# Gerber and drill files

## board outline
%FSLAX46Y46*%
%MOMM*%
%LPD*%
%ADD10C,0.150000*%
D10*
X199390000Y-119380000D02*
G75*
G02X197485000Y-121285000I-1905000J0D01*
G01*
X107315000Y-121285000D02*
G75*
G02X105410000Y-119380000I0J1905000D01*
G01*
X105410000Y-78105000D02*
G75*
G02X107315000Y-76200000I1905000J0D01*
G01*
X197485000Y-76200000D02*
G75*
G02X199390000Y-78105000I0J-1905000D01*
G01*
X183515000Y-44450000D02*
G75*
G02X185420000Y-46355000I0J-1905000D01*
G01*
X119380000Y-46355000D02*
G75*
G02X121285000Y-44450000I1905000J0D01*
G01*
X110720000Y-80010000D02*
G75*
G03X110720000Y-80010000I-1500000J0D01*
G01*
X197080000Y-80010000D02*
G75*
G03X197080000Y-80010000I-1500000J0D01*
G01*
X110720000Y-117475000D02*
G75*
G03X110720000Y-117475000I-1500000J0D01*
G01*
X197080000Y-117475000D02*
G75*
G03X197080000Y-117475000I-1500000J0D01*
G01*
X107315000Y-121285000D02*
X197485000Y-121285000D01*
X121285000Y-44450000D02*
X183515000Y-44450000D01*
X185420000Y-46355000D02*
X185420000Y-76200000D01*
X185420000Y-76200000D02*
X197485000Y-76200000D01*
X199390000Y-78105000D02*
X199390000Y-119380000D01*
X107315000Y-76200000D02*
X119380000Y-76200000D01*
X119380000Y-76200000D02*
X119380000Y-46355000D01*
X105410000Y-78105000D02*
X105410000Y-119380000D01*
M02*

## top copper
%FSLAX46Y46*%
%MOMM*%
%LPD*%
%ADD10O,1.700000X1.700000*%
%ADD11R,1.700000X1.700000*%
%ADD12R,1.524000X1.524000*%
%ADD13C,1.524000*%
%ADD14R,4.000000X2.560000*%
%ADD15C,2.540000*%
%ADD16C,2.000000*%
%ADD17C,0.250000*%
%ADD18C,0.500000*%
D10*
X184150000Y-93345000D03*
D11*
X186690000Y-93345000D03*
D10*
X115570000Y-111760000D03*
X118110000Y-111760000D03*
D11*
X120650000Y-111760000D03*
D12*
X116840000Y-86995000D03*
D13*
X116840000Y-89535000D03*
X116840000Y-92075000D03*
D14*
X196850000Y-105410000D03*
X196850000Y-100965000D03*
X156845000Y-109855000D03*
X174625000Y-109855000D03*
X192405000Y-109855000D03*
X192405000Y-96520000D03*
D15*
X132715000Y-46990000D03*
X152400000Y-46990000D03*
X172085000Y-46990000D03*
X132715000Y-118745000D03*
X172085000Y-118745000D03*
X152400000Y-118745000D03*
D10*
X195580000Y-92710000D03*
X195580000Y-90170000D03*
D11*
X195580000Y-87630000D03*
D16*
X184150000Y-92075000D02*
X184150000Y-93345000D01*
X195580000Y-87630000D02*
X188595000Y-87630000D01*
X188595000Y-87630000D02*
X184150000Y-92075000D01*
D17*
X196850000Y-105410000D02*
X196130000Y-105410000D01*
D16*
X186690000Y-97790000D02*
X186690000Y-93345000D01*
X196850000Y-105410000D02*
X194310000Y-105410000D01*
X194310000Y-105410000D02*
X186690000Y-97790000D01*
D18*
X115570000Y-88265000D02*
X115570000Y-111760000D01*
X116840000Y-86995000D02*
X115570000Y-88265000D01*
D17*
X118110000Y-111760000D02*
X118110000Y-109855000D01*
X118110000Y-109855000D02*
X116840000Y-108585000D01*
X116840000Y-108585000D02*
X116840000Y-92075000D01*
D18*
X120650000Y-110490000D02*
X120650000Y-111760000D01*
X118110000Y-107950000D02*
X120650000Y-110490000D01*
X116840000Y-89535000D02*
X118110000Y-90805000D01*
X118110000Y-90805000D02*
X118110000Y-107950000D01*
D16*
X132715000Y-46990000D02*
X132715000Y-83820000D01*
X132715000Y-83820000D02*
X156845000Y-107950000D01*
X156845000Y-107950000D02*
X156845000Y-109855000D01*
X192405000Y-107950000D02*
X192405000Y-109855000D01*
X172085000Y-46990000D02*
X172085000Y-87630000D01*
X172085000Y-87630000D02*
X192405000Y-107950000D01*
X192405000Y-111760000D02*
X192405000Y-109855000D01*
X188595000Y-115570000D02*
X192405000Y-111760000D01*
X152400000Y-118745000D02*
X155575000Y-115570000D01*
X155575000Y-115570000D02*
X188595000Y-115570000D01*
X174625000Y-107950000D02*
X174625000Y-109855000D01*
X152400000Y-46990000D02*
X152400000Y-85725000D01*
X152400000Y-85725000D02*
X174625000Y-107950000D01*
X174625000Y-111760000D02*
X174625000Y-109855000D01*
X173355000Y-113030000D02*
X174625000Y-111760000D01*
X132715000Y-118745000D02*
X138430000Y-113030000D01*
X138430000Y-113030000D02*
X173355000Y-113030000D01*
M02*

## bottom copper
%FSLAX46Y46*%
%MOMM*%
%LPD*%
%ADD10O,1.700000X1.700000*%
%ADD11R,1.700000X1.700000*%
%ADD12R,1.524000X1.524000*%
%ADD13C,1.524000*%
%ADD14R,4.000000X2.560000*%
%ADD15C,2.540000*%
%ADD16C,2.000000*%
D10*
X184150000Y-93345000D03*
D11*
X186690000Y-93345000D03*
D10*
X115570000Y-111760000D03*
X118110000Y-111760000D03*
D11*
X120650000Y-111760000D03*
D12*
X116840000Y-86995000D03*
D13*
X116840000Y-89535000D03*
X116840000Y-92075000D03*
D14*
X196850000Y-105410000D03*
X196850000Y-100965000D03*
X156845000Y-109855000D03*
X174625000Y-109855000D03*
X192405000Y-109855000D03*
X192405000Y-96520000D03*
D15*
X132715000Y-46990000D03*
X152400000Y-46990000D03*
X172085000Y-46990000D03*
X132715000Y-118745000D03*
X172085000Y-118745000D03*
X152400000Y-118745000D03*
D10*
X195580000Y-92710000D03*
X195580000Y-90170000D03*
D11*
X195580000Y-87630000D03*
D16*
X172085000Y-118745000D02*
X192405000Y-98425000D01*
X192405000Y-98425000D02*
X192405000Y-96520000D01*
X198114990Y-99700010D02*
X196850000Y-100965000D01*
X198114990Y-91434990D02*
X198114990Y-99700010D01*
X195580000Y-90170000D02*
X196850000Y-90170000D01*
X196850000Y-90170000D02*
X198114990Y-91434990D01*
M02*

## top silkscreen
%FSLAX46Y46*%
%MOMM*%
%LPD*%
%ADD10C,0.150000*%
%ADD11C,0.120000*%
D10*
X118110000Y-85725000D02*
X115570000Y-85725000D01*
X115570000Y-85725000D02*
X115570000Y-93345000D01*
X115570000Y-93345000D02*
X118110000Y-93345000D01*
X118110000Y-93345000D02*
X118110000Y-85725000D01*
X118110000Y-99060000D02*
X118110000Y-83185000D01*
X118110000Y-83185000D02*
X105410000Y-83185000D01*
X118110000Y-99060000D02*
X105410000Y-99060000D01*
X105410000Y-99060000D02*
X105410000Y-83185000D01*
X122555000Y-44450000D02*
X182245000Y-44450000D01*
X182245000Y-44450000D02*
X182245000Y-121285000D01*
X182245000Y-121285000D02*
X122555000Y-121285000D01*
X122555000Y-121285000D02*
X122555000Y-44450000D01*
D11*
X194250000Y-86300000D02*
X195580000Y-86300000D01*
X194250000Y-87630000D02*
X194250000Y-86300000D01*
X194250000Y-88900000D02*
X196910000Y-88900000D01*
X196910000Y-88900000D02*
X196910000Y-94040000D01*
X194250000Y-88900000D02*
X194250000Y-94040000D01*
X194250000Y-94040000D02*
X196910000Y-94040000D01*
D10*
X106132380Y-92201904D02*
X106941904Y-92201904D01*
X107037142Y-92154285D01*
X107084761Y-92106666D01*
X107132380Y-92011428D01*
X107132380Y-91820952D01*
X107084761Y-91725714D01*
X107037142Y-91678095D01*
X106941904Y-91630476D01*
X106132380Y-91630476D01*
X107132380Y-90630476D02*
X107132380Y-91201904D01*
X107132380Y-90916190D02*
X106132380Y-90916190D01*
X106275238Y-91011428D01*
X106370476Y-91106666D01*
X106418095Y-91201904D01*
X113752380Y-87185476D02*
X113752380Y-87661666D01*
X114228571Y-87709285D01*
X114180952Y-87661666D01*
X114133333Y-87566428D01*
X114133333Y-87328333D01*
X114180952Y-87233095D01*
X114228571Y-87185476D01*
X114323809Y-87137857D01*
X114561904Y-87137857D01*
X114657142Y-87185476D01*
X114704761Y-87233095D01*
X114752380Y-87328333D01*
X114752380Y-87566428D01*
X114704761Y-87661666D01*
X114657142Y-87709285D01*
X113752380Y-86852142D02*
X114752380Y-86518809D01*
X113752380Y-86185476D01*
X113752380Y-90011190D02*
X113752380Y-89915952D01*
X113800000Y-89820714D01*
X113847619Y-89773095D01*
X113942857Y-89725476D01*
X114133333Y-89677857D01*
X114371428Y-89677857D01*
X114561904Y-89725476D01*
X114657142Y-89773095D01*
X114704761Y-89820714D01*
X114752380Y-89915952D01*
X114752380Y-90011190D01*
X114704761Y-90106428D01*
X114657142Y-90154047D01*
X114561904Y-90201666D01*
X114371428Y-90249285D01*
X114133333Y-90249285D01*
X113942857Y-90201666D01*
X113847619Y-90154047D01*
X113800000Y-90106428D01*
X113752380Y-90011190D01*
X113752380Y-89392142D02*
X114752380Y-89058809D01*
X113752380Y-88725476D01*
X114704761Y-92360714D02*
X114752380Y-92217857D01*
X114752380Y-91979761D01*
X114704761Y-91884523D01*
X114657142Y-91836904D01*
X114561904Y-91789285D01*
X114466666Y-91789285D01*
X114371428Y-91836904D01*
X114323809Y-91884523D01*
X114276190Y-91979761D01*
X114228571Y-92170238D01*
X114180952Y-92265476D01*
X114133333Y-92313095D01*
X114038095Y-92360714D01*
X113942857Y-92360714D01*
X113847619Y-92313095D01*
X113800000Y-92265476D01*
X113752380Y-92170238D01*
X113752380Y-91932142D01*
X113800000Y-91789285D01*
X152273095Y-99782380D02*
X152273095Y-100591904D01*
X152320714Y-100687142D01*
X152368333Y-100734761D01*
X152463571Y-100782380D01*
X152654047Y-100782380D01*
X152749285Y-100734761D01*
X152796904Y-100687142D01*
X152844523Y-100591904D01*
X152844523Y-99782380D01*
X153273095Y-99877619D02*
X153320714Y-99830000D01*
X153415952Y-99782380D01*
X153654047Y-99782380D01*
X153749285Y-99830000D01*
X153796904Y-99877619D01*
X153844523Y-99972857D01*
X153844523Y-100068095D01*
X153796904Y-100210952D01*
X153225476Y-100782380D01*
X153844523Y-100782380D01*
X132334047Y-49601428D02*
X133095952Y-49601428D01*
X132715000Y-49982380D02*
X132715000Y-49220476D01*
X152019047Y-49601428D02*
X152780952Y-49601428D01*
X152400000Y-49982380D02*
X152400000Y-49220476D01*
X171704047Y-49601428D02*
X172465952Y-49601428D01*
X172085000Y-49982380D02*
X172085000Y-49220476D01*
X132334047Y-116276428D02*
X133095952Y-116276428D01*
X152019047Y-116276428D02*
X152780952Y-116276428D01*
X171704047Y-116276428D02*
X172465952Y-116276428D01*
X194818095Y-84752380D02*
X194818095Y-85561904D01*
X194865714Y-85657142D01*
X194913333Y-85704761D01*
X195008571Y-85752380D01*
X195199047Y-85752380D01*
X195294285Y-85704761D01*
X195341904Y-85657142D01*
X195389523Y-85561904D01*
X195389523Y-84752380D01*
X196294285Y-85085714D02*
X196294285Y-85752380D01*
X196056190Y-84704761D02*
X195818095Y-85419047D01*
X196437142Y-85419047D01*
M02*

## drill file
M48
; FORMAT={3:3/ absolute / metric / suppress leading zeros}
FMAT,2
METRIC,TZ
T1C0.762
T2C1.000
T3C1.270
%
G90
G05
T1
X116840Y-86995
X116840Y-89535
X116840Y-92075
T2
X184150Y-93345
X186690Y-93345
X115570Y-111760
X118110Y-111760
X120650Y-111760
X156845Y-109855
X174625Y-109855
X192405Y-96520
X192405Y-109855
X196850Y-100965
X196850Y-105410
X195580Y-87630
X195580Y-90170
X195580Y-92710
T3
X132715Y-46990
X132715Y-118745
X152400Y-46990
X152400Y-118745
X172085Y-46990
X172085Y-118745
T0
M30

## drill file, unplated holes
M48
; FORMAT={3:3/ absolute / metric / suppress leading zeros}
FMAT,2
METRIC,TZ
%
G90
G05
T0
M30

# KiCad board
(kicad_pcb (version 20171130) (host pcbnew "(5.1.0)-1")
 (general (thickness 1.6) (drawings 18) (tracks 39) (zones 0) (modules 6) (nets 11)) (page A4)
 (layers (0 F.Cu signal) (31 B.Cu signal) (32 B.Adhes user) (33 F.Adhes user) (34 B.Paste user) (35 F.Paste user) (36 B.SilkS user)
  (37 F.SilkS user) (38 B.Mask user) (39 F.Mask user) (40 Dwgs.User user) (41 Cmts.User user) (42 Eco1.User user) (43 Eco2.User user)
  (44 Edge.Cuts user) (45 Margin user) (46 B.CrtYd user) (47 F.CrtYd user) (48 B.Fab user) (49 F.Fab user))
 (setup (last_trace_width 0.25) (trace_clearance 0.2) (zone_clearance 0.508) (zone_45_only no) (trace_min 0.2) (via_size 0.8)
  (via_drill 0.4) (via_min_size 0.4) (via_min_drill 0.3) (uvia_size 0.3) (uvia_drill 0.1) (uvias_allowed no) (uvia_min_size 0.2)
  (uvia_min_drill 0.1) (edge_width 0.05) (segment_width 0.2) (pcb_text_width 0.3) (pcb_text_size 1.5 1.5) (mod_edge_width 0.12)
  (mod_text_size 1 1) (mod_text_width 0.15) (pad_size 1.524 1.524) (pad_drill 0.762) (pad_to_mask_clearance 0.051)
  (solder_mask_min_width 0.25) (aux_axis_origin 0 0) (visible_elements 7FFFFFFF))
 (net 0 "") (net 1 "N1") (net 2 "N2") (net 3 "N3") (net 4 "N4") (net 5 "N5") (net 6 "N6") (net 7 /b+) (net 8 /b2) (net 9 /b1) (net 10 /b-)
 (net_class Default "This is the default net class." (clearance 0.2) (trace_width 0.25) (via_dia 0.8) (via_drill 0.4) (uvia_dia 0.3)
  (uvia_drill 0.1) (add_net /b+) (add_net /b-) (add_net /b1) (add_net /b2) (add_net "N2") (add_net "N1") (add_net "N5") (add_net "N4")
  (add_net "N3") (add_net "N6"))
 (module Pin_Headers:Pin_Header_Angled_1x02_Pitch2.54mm (layer B.Cu) (at 186.69 93.345 90)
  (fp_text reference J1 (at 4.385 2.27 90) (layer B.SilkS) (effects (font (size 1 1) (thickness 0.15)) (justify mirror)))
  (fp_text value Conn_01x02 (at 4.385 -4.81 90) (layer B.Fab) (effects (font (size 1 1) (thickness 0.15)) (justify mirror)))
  (pad 2 thru_hole oval (at 0 -2.54 90) (size 1.7 1.7) (drill 1) (layers *.Cu *.Mask) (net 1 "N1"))
  (pad 1 thru_hole rect (at 0 0 90) (size 1.7 1.7) (drill 1) (layers *.Cu *.Mask) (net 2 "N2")))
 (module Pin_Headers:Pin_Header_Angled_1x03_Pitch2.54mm (layer B.Cu) (at 120.65 111.76 90)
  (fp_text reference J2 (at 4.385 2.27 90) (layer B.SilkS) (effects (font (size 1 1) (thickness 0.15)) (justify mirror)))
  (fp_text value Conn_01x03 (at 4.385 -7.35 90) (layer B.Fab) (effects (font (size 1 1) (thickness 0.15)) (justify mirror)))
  (pad 3 thru_hole oval (at 0 -5.08 90) (size 1.7 1.7) (drill 1) (layers *.Cu *.Mask) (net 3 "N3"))
  (pad 2 thru_hole oval (at 0 -2.54 90) (size 1.7 1.7) (drill 1) (layers *.Cu *.Mask) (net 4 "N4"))
  (pad 1 thru_hole rect (at 0 0 90) (size 1.7 1.7) (drill 1) (layers *.Cu *.Mask) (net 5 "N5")))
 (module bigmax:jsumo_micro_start (layer F.Cu) (at 116.84 86.995 270)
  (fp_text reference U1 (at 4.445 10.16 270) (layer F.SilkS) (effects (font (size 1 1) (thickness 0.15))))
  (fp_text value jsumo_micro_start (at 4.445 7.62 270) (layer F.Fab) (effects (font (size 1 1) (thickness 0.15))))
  (fp_line (start -1.27 -1.27) (end -1.27 1.27) (layer F.SilkS) (width 0.15))
  (fp_line (start -1.27 1.27) (end 6.35 1.27) (layer F.SilkS) (width 0.15))
  (fp_line (start 6.35 1.27) (end 6.35 -1.27) (layer F.SilkS) (width 0.15))
  (fp_line (start 6.35 -1.27) (end -1.27 -1.27) (layer F.SilkS) (width 0.15))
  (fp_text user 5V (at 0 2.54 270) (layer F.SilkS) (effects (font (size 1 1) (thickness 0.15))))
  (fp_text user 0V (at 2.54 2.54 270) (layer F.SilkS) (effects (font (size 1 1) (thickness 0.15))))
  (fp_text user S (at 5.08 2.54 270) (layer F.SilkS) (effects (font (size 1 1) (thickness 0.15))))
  (fp_line (start 12.065 -1.27) (end -3.81 -1.27) (layer F.SilkS) (width 0.15))
  (fp_line (start -3.81 -1.27) (end -3.81 11.43) (layer F.SilkS) (width 0.15))
  (fp_line (start 12.065 -1.27) (end 12.065 11.43) (layer F.SilkS) (width 0.15))
  (fp_line (start 12.065 11.43) (end -3.81 11.43) (layer F.SilkS) (width 0.15))
  (pad 1 thru_hole rect (at 0 0 270) (size 1.524 1.524) (drill 0.762) (layers *.Cu *.Mask) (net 3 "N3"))
  (pad 2 thru_hole circle (at 2.54 0 270) (size 1.524 1.524) (drill 0.762) (layers *.Cu *.Mask) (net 5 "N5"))
  (pad 3 thru_hole circle (at 5.08 0 270) (size 1.524 1.524) (drill 0.762) (layers *.Cu *.Mask) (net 4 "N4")))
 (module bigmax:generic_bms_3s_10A (layer B.Cu) (at 196.85 100.965)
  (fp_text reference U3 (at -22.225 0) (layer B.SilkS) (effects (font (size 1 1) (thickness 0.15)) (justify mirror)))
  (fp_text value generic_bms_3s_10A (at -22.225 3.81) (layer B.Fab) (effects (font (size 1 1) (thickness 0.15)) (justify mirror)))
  (pad 2 thru_hole rect (at 0 4.445) (size 4 2.56) (drill 1) (layers *.Cu *.Mask) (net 2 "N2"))
  (pad 1 thru_hole rect (at 0 0) (size 4 2.56) (drill 1) (layers *.Cu *.Mask) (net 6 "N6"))
  (pad 3 thru_hole rect (at -40.005 8.89) (size 4 2.56) (drill 1) (layers *.Cu *.Mask) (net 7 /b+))
  (pad 5 thru_hole rect (at -22.225 8.89) (size 4 2.56) (drill 1) (layers *.Cu *.Mask) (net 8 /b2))
  (pad 4 thru_hole rect (at -4.445 8.89) (size 4 2.56) (drill 1) (layers *.Cu *.Mask) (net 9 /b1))
  (pad 6 thru_hole rect (at -4.445 -4.445) (size 4 2.56) (drill 1) (layers *.Cu *.Mask) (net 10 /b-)))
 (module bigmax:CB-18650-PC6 (layer F.Cu) (at 132.715 46.99)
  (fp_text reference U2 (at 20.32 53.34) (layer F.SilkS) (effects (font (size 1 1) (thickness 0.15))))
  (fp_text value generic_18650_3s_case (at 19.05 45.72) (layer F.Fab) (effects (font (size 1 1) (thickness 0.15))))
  (fp_line (start -10.16 -2.54) (end 49.53 -2.54) (layer F.SilkS) (width 0.15))
  (fp_line (start 49.53 -2.54) (end 49.53 74.295) (layer F.SilkS) (width 0.15))
  (fp_line (start 49.53 74.295) (end -10.16 74.295) (layer F.SilkS) (width 0.15))
  (fp_line (start -10.16 74.295) (end -10.16 -2.54) (layer F.SilkS) (width 0.15))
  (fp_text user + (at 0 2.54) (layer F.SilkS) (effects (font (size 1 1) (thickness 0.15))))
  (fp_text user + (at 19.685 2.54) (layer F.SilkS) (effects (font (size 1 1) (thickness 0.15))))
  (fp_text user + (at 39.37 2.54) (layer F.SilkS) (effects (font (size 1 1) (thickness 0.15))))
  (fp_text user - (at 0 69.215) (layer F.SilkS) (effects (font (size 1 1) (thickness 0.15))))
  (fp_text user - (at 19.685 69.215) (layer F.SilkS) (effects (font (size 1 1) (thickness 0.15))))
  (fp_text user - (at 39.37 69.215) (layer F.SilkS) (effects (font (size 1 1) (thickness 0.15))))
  (pad 1 thru_hole circle (at 0 0) (size 2.54 2.54) (drill 1.27) (layers *.Cu *.Mask) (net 7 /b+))
  (pad 2 thru_hole circle (at 19.685 0) (size 2.54 2.54) (drill 1.27) (layers *.Cu *.Mask) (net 8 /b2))
  (pad 3 thru_hole circle (at 39.37 0) (size 2.54 2.54) (drill 1.27) (layers *.Cu *.Mask) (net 9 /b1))
  (pad 4 thru_hole circle (at 0 71.755) (size 2.54 2.54) (drill 1.27) (layers *.Cu *.Mask) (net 8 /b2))
  (pad 6 thru_hole circle (at 39.37 71.755) (size 2.54 2.54) (drill 1.27) (layers *.Cu *.Mask) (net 10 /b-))
  (pad 5 thru_hole circle (at 19.685 71.755) (size 2.54 2.54) (drill 1.27) (layers *.Cu *.Mask) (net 9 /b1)))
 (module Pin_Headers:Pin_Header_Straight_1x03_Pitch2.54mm (layer F.Cu) (at 195.58 87.63)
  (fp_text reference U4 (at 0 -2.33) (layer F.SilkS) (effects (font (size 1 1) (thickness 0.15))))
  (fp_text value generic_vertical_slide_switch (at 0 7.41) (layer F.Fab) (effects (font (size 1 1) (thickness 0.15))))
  (fp_line (start -1.33 -1.33) (end 0 -1.33) (layer F.SilkS) (width 0.12))
  (fp_line (start -1.33 0) (end -1.33 -1.33) (layer F.SilkS) (width 0.12))
  (fp_line (start -1.33 1.27) (end 1.33 1.27) (layer F.SilkS) (width 0.12))
  (fp_line (start 1.33 1.27) (end 1.33 6.41) (layer F.SilkS) (width 0.12))
  (fp_line (start -1.33 1.27) (end -1.33 6.41) (layer F.SilkS) (width 0.12))
  (fp_line (start -1.33 6.41) (end 1.33 6.41) (layer F.SilkS) (width 0.12))
  (pad 3 thru_hole oval (at 0 5.08) (size 1.7 1.7) (drill 1) (layers *.Cu *.Mask))
  (pad 2 thru_hole oval (at 0 2.54) (size 1.7 1.7) (drill 1) (layers *.Cu *.Mask) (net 6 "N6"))
  (pad 1 thru_hole rect (at 0 0) (size 1.7 1.7) (drill 1) (layers *.Cu *.Mask) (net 1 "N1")))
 (gr_arc (start 197.485 119.38) (end 197.485 121.285) (angle -90) (layer Edge.Cuts) (width 0.15))
 (gr_arc (start 107.315 119.38) (end 105.41 119.38) (angle -90) (layer Edge.Cuts) (width 0.15))
 (gr_arc (start 107.315 78.105) (end 107.315 76.2) (angle -90) (layer Edge.Cuts) (width 0.15))
 (gr_arc (start 197.485 78.105) (end 199.39 78.105) (angle -90) (layer Edge.Cuts) (width 0.15))
 (gr_arc (start 183.515 46.355) (end 185.42 46.355) (angle -90) (layer Edge.Cuts) (width 0.15))
 (gr_arc (start 121.285 46.355) (end 121.285 44.45) (angle -90) (layer Edge.Cuts) (width 0.15))
 (gr_circle (center 109.22 80.01) (end 110.72 80.01) (layer Edge.Cuts) (width 0.15))
 (gr_circle (center 195.58 80.01) (end 197.08 80.01) (layer Edge.Cuts) (width 0.15))
 (gr_circle (center 109.22 117.475) (end 110.72 117.475) (layer Edge.Cuts) (width 0.15))
 (gr_circle (center 195.58 117.475) (end 197.08 117.475) (layer Edge.Cuts) (width 0.15))
 (gr_line (start 107.315 121.285) (end 197.485 121.285) (layer Edge.Cuts) (width 0.15))
 (gr_line (start 121.285 44.45) (end 183.515 44.45) (layer Edge.Cuts) (width 0.15))
 (gr_line (start 185.42 46.355) (end 185.42 76.2) (layer Edge.Cuts) (width 0.15))
 (gr_line (start 185.42 76.2) (end 197.485 76.2) (layer Edge.Cuts) (width 0.15))
 (gr_line (start 199.39 78.105) (end 199.39 119.38) (layer Edge.Cuts) (width 0.15))
 (gr_line (start 107.315 76.2) (end 119.38 76.2) (layer Edge.Cuts) (width 0.15))
 (gr_line (start 119.38 76.2) (end 119.38 46.355) (layer Edge.Cuts) (width 0.15))
 (gr_line (start 105.41 78.105) (end 105.41 119.38) (layer Edge.Cuts) (width 0.15))
 (segment (start 184.15 92.075) (end 184.15 93.345) (width 2) (layer F.Cu) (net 1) (status 20))
 (segment (start 195.58 87.63) (end 188.595 87.63) (width 2) (layer F.Cu) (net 1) (status 10))
 (segment (start 188.595 87.63) (end 184.15 92.075) (width 2) (layer F.Cu) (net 1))
 (segment (start 196.85 105.41) (end 196.13 105.41) (width 0.25) (layer F.Cu) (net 2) (status 30))
 (segment (start 186.69 97.79) (end 186.69 93.345) (width 2) (layer F.Cu) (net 2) (status 20))
 (segment (start 196.85 105.41) (end 194.31 105.41) (width 2) (layer F.Cu) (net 2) (status 10))
 (segment (start 194.31 105.41) (end 186.69 97.79) (width 2) (layer F.Cu) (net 2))
 (segment (start 115.57 88.265) (end 115.57 111.76) (width 0.5) (layer F.Cu) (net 3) (status 20))
 (segment (start 116.84 86.995) (end 115.57 88.265) (width 0.5) (layer F.Cu) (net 3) (status 10))
 (segment (start 118.11 111.76) (end 118.11 109.855) (width 0.25) (layer F.Cu) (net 4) (status 10))
 (segment (start 118.11 109.855) (end 116.84 108.585) (width 0.25) (layer F.Cu) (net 4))
 (segment (start 116.84 108.585) (end 116.84 92.075) (width 0.25) (layer F.Cu) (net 4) (status 20))
 (segment (start 120.65 110.49) (end 120.65 111.76) (width 0.5) (layer F.Cu) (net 5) (status 20))
 (segment (start 118.11 107.95) (end 120.65 110.49) (width 0.5) (layer F.Cu) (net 5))
 (segment (start 116.84 89.535) (end 118.11 90.805) (width 0.5) (layer F.Cu) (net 5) (status 10))
 (segment (start 118.11 90.805) (end 118.11 107.95) (width 0.5) (layer F.Cu) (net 5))
 (segment (start 132.715 46.99) (end 132.715 83.82) (width 2) (layer F.Cu) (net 7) (status 10))
 (segment (start 132.715 83.82) (end 156.845 107.95) (width 2) (layer F.Cu) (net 7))
 (segment (start 156.845 107.95) (end 156.845 109.855) (width 2) (layer F.Cu) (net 7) (status 20))
 (segment (start 192.405 107.95) (end 192.405 109.855) (width 2) (layer F.Cu) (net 9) (status 20))
 (segment (start 172.085 46.99) (end 172.085 87.63) (width 2) (layer F.Cu) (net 9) (status 10))
 (segment (start 172.085 87.63) (end 192.405 107.95) (width 2) (layer F.Cu) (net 9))
 (segment (start 192.405 111.76) (end 192.405 109.855) (width 2) (layer F.Cu) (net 9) (status 20))
 (segment (start 188.595 115.57) (end 192.405 111.76) (width 2) (layer F.Cu) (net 9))
 (segment (start 152.4 118.745) (end 155.575 115.57) (width 2) (layer F.Cu) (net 9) (status 10))
 (segment (start 155.575 115.57) (end 188.595 115.57) (width 2) (layer F.Cu) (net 9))
 (segment (start 174.625 107.95) (end 174.625 109.855) (width 2) (layer F.Cu) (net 8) (status 20))
 (segment (start 152.4 46.99) (end 152.4 85.725) (width 2) (layer F.Cu) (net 8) (status 10))
 (segment (start 152.4 85.725) (end 174.625 107.95) (width 2) (layer F.Cu) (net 8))
 (segment (start 174.625 111.76) (end 174.625 109.855) (width 2) (layer F.Cu) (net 8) (status 20))
 (segment (start 173.355 113.03) (end 174.625 111.76) (width 2) (layer F.Cu) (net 8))
 (segment (start 132.715 118.745) (end 138.43 113.03) (width 2) (layer F.Cu) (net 8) (status 10))
 (segment (start 138.43 113.03) (end 173.355 113.03) (width 2) (layer F.Cu) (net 8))
 (segment (start 172.085 118.745) (end 192.405 98.425) (width 2) (layer B.Cu) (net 10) (status 10))
 (segment (start 192.405 98.425) (end 192.405 96.52) (width 2) (layer B.Cu) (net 10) (status 20))
 (segment (start 198.11499 99.70001) (end 196.85 100.965) (width 2) (layer B.Cu) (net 6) (status 30))
 (segment (start 198.11499 91.43499) (end 198.11499 99.70001) (width 2) (layer B.Cu) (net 6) (status 20))
 (segment (start 195.58 90.17) (end 196.85 90.17) (width 2) (layer B.Cu) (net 6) (status 10))
 (segment (start 196.85 90.17) (end 198.11499 91.43499) (width 2) (layer B.Cu) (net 6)))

